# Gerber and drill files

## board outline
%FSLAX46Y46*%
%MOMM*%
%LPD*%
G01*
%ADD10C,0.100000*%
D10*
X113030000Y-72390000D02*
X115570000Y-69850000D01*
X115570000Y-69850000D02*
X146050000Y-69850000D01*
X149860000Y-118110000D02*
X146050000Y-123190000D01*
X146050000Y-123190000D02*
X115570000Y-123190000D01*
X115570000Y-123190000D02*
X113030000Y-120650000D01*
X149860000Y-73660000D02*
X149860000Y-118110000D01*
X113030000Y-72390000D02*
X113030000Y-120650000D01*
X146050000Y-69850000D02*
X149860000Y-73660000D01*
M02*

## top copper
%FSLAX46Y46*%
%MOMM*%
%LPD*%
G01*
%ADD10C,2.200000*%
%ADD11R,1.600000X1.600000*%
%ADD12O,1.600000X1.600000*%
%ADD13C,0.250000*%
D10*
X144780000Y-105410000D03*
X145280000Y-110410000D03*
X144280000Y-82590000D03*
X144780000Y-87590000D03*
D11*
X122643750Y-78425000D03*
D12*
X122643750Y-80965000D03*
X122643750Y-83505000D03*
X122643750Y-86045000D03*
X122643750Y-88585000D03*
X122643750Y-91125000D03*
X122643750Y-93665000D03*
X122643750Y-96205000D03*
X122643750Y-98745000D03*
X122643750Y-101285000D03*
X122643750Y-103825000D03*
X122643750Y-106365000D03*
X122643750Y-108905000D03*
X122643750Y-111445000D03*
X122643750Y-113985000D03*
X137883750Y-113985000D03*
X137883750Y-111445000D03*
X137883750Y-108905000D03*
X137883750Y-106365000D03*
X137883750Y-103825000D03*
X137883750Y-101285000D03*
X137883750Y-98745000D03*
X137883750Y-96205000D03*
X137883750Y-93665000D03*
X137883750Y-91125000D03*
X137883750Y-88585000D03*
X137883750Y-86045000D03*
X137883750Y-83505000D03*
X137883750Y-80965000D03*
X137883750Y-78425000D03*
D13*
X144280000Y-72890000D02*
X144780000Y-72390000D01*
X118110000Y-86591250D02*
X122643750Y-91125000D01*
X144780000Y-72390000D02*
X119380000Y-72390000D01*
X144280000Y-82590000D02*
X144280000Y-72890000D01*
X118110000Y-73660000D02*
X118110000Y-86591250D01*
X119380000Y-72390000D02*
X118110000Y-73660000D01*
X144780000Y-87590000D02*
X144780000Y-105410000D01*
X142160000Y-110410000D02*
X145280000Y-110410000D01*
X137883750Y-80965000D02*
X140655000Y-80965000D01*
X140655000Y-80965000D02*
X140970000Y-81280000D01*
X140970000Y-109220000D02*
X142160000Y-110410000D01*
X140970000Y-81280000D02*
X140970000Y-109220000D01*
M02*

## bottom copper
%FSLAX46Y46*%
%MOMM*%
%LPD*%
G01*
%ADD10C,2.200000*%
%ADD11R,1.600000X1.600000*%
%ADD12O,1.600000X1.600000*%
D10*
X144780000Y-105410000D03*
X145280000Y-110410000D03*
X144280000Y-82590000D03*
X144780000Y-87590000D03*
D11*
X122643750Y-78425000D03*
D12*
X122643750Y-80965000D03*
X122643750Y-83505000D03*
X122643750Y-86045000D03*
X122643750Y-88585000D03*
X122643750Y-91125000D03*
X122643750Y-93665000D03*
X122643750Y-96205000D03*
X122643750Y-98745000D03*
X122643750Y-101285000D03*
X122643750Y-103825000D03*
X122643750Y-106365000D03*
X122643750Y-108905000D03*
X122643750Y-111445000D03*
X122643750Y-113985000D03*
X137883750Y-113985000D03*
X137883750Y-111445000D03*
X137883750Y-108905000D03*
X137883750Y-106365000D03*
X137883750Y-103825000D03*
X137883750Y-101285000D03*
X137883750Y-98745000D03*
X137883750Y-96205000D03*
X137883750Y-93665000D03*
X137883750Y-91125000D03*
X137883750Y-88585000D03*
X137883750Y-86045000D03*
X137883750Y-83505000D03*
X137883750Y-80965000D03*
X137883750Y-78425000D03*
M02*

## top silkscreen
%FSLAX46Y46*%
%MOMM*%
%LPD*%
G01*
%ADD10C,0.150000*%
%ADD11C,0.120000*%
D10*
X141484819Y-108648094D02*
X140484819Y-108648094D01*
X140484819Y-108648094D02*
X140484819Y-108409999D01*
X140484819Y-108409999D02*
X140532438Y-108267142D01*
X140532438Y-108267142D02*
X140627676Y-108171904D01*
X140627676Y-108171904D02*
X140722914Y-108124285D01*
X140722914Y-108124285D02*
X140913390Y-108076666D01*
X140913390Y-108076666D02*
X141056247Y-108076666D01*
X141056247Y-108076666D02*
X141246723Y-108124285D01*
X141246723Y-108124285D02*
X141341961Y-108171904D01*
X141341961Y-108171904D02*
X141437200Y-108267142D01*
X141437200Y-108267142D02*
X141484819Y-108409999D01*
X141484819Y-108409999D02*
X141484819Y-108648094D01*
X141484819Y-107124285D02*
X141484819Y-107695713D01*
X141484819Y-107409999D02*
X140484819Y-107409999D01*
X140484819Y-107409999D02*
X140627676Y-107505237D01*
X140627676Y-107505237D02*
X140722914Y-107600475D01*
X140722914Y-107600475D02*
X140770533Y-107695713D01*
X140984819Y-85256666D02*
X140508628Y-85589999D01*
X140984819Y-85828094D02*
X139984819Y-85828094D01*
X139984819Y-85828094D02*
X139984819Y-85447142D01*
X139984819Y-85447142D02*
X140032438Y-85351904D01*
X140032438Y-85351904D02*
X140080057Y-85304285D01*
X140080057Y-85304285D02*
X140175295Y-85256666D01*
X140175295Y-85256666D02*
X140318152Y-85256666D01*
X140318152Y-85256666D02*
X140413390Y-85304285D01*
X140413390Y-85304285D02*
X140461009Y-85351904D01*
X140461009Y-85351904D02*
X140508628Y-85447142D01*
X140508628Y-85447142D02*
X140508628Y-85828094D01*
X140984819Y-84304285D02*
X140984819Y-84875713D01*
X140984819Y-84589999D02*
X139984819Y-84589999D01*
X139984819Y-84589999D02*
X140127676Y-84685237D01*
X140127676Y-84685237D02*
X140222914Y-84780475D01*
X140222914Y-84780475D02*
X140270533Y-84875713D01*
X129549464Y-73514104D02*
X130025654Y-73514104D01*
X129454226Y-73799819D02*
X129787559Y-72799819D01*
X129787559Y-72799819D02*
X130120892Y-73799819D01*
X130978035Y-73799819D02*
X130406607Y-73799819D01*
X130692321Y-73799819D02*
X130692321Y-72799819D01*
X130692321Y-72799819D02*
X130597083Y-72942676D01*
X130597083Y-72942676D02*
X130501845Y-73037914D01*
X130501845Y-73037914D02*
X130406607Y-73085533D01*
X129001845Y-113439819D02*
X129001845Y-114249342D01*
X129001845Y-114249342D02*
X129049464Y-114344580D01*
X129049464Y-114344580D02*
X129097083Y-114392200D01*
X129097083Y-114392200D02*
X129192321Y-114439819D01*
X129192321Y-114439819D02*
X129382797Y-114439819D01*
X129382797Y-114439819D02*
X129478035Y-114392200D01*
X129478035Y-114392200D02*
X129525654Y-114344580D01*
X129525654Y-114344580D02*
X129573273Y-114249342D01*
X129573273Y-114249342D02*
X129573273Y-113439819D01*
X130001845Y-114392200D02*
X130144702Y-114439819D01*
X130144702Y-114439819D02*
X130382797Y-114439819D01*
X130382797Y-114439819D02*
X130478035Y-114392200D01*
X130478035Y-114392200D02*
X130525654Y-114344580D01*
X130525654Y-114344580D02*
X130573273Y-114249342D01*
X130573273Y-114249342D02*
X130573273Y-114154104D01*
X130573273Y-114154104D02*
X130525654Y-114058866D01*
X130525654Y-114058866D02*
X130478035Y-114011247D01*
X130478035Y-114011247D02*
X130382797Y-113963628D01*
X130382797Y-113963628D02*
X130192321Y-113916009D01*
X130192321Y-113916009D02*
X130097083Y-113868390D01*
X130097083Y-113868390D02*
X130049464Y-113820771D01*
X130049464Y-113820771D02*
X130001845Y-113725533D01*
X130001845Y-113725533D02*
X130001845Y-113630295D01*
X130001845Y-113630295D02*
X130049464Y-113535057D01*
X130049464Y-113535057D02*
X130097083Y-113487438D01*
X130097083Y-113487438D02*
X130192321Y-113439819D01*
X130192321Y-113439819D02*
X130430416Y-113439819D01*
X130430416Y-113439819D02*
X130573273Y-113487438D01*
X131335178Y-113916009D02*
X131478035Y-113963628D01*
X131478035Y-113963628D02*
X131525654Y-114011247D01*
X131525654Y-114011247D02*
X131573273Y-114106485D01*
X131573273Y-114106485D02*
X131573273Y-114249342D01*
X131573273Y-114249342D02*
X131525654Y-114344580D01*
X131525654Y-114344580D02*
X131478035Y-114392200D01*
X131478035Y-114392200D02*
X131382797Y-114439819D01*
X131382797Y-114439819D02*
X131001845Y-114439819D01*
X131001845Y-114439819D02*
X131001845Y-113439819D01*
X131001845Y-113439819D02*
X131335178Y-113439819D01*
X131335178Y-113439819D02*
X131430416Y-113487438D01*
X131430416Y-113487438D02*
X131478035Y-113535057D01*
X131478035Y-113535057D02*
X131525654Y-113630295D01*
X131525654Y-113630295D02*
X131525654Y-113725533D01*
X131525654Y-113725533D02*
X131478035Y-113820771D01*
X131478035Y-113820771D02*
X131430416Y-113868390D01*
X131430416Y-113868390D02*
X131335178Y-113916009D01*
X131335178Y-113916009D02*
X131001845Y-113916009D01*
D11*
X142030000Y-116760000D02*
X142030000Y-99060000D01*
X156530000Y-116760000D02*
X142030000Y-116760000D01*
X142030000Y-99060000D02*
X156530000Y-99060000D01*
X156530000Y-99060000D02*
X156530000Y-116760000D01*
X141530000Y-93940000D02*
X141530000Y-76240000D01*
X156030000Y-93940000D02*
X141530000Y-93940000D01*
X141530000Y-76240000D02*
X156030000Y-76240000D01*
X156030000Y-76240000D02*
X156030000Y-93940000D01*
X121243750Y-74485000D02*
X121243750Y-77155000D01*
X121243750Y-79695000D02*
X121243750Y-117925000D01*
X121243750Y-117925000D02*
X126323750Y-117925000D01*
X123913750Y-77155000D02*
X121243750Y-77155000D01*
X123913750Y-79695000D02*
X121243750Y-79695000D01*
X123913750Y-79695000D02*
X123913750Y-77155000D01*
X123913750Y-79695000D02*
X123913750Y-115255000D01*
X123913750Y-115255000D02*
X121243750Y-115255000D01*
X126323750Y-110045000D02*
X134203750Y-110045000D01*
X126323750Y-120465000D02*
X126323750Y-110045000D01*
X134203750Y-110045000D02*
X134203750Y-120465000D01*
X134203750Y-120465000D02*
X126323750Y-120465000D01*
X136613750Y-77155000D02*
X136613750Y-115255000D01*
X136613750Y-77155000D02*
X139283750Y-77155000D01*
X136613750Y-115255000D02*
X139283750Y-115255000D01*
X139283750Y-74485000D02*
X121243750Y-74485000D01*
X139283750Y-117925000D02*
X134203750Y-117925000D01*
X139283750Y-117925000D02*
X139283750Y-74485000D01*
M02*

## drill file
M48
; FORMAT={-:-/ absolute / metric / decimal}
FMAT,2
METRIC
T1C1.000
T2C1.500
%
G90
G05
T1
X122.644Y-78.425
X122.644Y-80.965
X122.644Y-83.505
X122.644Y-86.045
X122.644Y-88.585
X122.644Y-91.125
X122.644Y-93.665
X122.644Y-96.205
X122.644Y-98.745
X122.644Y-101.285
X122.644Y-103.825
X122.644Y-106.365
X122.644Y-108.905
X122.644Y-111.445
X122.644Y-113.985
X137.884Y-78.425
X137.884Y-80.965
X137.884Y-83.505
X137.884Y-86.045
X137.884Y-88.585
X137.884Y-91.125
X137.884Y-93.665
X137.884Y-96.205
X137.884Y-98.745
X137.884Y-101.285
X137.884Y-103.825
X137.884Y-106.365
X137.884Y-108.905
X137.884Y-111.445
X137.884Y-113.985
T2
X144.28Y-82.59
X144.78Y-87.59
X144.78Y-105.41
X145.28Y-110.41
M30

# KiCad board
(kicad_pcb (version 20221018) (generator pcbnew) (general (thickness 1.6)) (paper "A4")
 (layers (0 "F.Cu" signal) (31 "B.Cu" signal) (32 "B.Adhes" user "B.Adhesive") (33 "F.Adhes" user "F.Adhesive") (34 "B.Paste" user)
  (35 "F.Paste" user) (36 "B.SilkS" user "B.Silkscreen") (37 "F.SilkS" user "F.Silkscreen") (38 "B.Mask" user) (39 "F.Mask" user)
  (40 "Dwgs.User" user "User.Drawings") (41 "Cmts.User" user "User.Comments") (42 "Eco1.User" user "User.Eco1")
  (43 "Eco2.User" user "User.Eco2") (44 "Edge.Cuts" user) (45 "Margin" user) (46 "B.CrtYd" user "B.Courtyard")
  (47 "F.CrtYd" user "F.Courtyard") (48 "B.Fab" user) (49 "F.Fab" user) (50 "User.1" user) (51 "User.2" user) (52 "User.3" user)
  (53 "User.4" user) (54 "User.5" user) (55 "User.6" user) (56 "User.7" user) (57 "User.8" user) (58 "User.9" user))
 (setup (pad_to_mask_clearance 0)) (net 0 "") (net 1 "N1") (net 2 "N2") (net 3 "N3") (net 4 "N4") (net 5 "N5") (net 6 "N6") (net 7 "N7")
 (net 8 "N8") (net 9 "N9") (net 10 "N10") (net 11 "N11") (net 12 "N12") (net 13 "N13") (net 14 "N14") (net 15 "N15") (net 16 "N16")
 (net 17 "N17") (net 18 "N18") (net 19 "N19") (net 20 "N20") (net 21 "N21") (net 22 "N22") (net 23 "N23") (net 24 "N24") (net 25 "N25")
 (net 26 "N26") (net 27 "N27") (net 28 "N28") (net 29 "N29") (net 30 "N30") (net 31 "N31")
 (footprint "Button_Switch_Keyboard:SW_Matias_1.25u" (layer "F.Cu") (at 144.78 105.41 90)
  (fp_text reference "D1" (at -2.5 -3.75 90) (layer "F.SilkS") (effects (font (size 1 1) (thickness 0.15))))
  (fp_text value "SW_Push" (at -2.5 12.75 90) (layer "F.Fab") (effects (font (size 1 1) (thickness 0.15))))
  (fp_line (start -11.35 -2.75) (end 6.35 -2.75) (stroke (width 0.12) (type solid)) (layer "F.SilkS"))
  (fp_line (start -11.35 11.75) (end -11.35 -2.75) (stroke (width 0.12) (type solid)) (layer "F.SilkS"))
  (fp_line (start 6.35 -2.75) (end 6.35 11.75) (stroke (width 0.12) (type solid)) (layer "F.SilkS"))
  (fp_line (start 6.35 11.75) (end -11.35 11.75) (stroke (width 0.12) (type solid)) (layer "F.SilkS"))
  (pad "1" thru_hole circle (at 0 0 90) (size 2.2 2.2) (drill 1.5) (layers "*.Cu" "*.Mask") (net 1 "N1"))
  (pad "2" thru_hole circle (at -5 0.5 90) (size 2.2 2.2) (drill 1.5) (layers "*.Cu" "*.Mask") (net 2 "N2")))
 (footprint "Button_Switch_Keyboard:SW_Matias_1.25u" (layer "F.Cu") (at 144.28 82.59 90)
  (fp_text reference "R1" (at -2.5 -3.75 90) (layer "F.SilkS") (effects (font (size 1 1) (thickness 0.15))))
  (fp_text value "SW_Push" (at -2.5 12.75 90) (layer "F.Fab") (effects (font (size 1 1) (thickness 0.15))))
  (fp_line (start -11.35 -2.75) (end 6.35 -2.75) (stroke (width 0.12) (type solid)) (layer "F.SilkS"))
  (fp_line (start -11.35 11.75) (end -11.35 -2.75) (stroke (width 0.12) (type solid)) (layer "F.SilkS"))
  (fp_line (start 6.35 -2.75) (end 6.35 11.75) (stroke (width 0.12) (type solid)) (layer "F.SilkS"))
  (fp_line (start 6.35 11.75) (end -11.35 11.75) (stroke (width 0.12) (type solid)) (layer "F.SilkS"))
  (pad "1" thru_hole circle (at 0 0 90) (size 2.2 2.2) (drill 1.5) (layers "*.Cu" "*.Mask") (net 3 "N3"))
  (pad "2" thru_hole circle (at -5 0.5 90) (size 2.2 2.2) (drill 1.5) (layers "*.Cu" "*.Mask") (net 1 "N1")))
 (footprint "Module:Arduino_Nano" (layer "F.Cu") (at 122.64375 78.425)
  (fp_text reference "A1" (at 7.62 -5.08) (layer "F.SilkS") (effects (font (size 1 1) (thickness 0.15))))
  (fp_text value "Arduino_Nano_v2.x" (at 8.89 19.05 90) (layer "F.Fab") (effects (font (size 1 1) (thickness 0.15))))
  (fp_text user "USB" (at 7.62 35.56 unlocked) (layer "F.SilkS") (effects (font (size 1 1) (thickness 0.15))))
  (fp_line (start -1.4 -3.94) (end -1.4 -1.27) (stroke (width 0.12) (type solid)) (layer "F.SilkS"))
  (fp_line (start -1.4 1.27) (end -1.4 39.5) (stroke (width 0.12) (type solid)) (layer "F.SilkS"))
  (fp_line (start -1.4 39.5) (end 3.68 39.5) (stroke (width 0.12) (type solid)) (layer "F.SilkS"))
  (fp_line (start 1.27 -1.27) (end -1.4 -1.27) (stroke (width 0.12) (type solid)) (layer "F.SilkS"))
  (fp_line (start 1.27 1.27) (end -1.4 1.27) (stroke (width 0.12) (type solid)) (layer "F.SilkS"))
  (fp_line (start 1.27 1.27) (end 1.27 -1.27) (stroke (width 0.12) (type solid)) (layer "F.SilkS"))
  (fp_line (start 1.27 1.27) (end 1.27 36.83) (stroke (width 0.12) (type solid)) (layer "F.SilkS"))
  (fp_line (start 1.27 36.83) (end -1.4 36.83) (stroke (width 0.12) (type solid)) (layer "F.SilkS"))
  (fp_line (start 3.68 31.62) (end 11.56 31.62) (stroke (width 0.12) (type solid)) (layer "F.SilkS"))
  (fp_line (start 3.68 42.04) (end 3.68 31.62) (stroke (width 0.12) (type solid)) (layer "F.SilkS"))
  (fp_line (start 11.56 31.62) (end 11.56 42.04) (stroke (width 0.12) (type solid)) (layer "F.SilkS"))
  (fp_line (start 11.56 42.04) (end 3.68 42.04) (stroke (width 0.12) (type solid)) (layer "F.SilkS"))
  (fp_line (start 13.97 -1.27) (end 13.97 36.83) (stroke (width 0.12) (type solid)) (layer "F.SilkS"))
  (fp_line (start 13.97 -1.27) (end 16.64 -1.27) (stroke (width 0.12) (type solid)) (layer "F.SilkS"))
  (fp_line (start 13.97 36.83) (end 16.64 36.83) (stroke (width 0.12) (type solid)) (layer "F.SilkS"))
  (fp_line (start 16.64 -3.94) (end -1.4 -3.94) (stroke (width 0.12) (type solid)) (layer "F.SilkS"))
  (fp_line (start 16.64 39.5) (end 11.56 39.5) (stroke (width 0.12) (type solid)) (layer "F.SilkS"))
  (fp_line (start 16.64 39.5) (end 16.64 -3.94) (stroke (width 0.12) (type solid)) (layer "F.SilkS"))
  (pad "1" thru_hole rect (at 0 0) (size 1.6 1.6) (drill 1) (layers "*.Cu" "*.Mask") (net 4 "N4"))
  (pad "2" thru_hole oval (at 0 2.54) (size 1.6 1.6) (drill 1) (layers "*.Cu" "*.Mask") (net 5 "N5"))
  (pad "3" thru_hole oval (at 0 5.08) (size 1.6 1.6) (drill 1) (layers "*.Cu" "*.Mask") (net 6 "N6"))
  (pad "4" thru_hole oval (at 0 7.62) (size 1.6 1.6) (drill 1) (layers "*.Cu" "*.Mask") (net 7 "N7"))
  (pad "5" thru_hole oval (at 0 10.16) (size 1.6 1.6) (drill 1) (layers "*.Cu" "*.Mask") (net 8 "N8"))
  (pad "6" thru_hole oval (at 0 12.7) (size 1.6 1.6) (drill 1) (layers "*.Cu" "*.Mask") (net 3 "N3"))
  (pad "7" thru_hole oval (at 0 15.24) (size 1.6 1.6) (drill 1) (layers "*.Cu" "*.Mask") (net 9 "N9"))
  (pad "8" thru_hole oval (at 0 17.78) (size 1.6 1.6) (drill 1) (layers "*.Cu" "*.Mask") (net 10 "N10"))
  (pad "9" thru_hole oval (at 0 20.32) (size 1.6 1.6) (drill 1) (layers "*.Cu" "*.Mask") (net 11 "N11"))
  (pad "10" thru_hole oval (at 0 22.86) (size 1.6 1.6) (drill 1) (layers "*.Cu" "*.Mask") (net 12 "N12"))
  (pad "11" thru_hole oval (at 0 25.4) (size 1.6 1.6) (drill 1) (layers "*.Cu" "*.Mask") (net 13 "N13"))
  (pad "12" thru_hole oval (at 0 27.94) (size 1.6 1.6) (drill 1) (layers "*.Cu" "*.Mask") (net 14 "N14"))
  (pad "13" thru_hole oval (at 0 30.48) (size 1.6 1.6) (drill 1) (layers "*.Cu" "*.Mask") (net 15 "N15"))
  (pad "14" thru_hole oval (at 0 33.02) (size 1.6 1.6) (drill 1) (layers "*.Cu" "*.Mask") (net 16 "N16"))
  (pad "15" thru_hole oval (at 0 35.56) (size 1.6 1.6) (drill 1) (layers "*.Cu" "*.Mask") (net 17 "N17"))
  (pad "16" thru_hole oval (at 15.24 35.56) (size 1.6 1.6) (drill 1) (layers "*.Cu" "*.Mask") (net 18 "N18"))
  (pad "17" thru_hole oval (at 15.24 33.02) (size 1.6 1.6) (drill 1) (layers "*.Cu" "*.Mask") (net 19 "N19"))
  (pad "18" thru_hole oval (at 15.24 30.48) (size 1.6 1.6) (drill 1) (layers "*.Cu" "*.Mask") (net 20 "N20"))
  (pad "19" thru_hole oval (at 15.24 27.94) (size 1.6 1.6) (drill 1) (layers "*.Cu" "*.Mask") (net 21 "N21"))
  (pad "20" thru_hole oval (at 15.24 25.4) (size 1.6 1.6) (drill 1) (layers "*.Cu" "*.Mask") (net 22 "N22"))
  (pad "21" thru_hole oval (at 15.24 22.86) (size 1.6 1.6) (drill 1) (layers "*.Cu" "*.Mask") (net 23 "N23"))
  (pad "22" thru_hole oval (at 15.24 20.32) (size 1.6 1.6) (drill 1) (layers "*.Cu" "*.Mask") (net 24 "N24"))
  (pad "23" thru_hole oval (at 15.24 17.78) (size 1.6 1.6) (drill 1) (layers "*.Cu" "*.Mask") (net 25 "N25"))
  (pad "24" thru_hole oval (at 15.24 15.24) (size 1.6 1.6) (drill 1) (layers "*.Cu" "*.Mask") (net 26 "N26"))
  (pad "25" thru_hole oval (at 15.24 12.7) (size 1.6 1.6) (drill 1) (layers "*.Cu" "*.Mask") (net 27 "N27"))
  (pad "26" thru_hole oval (at 15.24 10.16) (size 1.6 1.6) (drill 1) (layers "*.Cu" "*.Mask") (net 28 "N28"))
  (pad "27" thru_hole oval (at 15.24 7.62) (size 1.6 1.6) (drill 1) (layers "*.Cu" "*.Mask") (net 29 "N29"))
  (pad "28" thru_hole oval (at 15.24 5.08) (size 1.6 1.6) (drill 1) (layers "*.Cu" "*.Mask") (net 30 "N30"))
  (pad "29" thru_hole oval (at 15.24 2.54) (size 1.6 1.6) (drill 1) (layers "*.Cu" "*.Mask") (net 2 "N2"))
  (pad "30" thru_hole oval (at 15.24 0) (size 1.6 1.6) (drill 1) (layers "*.Cu" "*.Mask") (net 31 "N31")))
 (gr_line (start 113.03 72.39) (end 115.57 69.85) (stroke (width 0.1) (type default)) (layer "Edge.Cuts"))
 (gr_line (start 115.57 69.85) (end 146.05 69.85) (stroke (width 0.1) (type default)) (layer "Edge.Cuts"))
 (gr_line (start 149.86 118.11) (end 146.05 123.19) (stroke (width 0.1) (type default)) (layer "Edge.Cuts"))
 (gr_line (start 146.05 123.19) (end 115.57 123.19) (stroke (width 0.1) (type default)) (layer "Edge.Cuts"))
 (gr_line (start 115.57 123.19) (end 113.03 120.65) (stroke (width 0.1) (type default)) (layer "Edge.Cuts"))
 (gr_line (start 149.86 73.66) (end 149.86 118.11) (stroke (width 0.1) (type default)) (layer "Edge.Cuts"))
 (gr_line (start 113.03 72.39) (end 113.03 120.65) (stroke (width 0.1) (type default)) (layer "Edge.Cuts"))
 (gr_line (start 146.05 69.85) (end 149.86 73.66) (stroke (width 0.1) (type default)) (layer "Edge.Cuts"))
 (segment (start 144.28 72.89) (end 144.78 72.39) (width 0.25) (layer "F.Cu") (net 3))
 (segment (start 118.11 86.59125) (end 122.64375 91.125) (width 0.25) (layer "F.Cu") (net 3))
 (segment (start 144.78 72.39) (end 119.38 72.39) (width 0.25) (layer "F.Cu") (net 3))
 (segment (start 144.28 82.59) (end 144.28 72.89) (width 0.25) (layer "F.Cu") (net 3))
 (segment (start 118.11 73.66) (end 118.11 86.59125) (width 0.25) (layer "F.Cu") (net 3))
 (segment (start 119.38 72.39) (end 118.11 73.66) (width 0.25) (layer "F.Cu") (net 3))
 (segment (start 144.78 87.59) (end 144.78 105.41) (width 0.25) (layer "F.Cu") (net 1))
 (segment (start 142.16 110.41) (end 145.28 110.41) (width 0.25) (layer "F.Cu") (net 2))
 (segment (start 137.88375 80.965) (end 140.655 80.965) (width 0.25) (layer "F.Cu") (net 2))
 (segment (start 140.655 80.965) (end 140.97 81.28) (width 0.25) (layer "F.Cu") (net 2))
 (segment (start 140.97 109.22) (end 142.16 110.41) (width 0.25) (layer "F.Cu") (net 2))
 (segment (start 140.97 81.28) (end 140.97 109.22) (width 0.25) (layer "F.Cu") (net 2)))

